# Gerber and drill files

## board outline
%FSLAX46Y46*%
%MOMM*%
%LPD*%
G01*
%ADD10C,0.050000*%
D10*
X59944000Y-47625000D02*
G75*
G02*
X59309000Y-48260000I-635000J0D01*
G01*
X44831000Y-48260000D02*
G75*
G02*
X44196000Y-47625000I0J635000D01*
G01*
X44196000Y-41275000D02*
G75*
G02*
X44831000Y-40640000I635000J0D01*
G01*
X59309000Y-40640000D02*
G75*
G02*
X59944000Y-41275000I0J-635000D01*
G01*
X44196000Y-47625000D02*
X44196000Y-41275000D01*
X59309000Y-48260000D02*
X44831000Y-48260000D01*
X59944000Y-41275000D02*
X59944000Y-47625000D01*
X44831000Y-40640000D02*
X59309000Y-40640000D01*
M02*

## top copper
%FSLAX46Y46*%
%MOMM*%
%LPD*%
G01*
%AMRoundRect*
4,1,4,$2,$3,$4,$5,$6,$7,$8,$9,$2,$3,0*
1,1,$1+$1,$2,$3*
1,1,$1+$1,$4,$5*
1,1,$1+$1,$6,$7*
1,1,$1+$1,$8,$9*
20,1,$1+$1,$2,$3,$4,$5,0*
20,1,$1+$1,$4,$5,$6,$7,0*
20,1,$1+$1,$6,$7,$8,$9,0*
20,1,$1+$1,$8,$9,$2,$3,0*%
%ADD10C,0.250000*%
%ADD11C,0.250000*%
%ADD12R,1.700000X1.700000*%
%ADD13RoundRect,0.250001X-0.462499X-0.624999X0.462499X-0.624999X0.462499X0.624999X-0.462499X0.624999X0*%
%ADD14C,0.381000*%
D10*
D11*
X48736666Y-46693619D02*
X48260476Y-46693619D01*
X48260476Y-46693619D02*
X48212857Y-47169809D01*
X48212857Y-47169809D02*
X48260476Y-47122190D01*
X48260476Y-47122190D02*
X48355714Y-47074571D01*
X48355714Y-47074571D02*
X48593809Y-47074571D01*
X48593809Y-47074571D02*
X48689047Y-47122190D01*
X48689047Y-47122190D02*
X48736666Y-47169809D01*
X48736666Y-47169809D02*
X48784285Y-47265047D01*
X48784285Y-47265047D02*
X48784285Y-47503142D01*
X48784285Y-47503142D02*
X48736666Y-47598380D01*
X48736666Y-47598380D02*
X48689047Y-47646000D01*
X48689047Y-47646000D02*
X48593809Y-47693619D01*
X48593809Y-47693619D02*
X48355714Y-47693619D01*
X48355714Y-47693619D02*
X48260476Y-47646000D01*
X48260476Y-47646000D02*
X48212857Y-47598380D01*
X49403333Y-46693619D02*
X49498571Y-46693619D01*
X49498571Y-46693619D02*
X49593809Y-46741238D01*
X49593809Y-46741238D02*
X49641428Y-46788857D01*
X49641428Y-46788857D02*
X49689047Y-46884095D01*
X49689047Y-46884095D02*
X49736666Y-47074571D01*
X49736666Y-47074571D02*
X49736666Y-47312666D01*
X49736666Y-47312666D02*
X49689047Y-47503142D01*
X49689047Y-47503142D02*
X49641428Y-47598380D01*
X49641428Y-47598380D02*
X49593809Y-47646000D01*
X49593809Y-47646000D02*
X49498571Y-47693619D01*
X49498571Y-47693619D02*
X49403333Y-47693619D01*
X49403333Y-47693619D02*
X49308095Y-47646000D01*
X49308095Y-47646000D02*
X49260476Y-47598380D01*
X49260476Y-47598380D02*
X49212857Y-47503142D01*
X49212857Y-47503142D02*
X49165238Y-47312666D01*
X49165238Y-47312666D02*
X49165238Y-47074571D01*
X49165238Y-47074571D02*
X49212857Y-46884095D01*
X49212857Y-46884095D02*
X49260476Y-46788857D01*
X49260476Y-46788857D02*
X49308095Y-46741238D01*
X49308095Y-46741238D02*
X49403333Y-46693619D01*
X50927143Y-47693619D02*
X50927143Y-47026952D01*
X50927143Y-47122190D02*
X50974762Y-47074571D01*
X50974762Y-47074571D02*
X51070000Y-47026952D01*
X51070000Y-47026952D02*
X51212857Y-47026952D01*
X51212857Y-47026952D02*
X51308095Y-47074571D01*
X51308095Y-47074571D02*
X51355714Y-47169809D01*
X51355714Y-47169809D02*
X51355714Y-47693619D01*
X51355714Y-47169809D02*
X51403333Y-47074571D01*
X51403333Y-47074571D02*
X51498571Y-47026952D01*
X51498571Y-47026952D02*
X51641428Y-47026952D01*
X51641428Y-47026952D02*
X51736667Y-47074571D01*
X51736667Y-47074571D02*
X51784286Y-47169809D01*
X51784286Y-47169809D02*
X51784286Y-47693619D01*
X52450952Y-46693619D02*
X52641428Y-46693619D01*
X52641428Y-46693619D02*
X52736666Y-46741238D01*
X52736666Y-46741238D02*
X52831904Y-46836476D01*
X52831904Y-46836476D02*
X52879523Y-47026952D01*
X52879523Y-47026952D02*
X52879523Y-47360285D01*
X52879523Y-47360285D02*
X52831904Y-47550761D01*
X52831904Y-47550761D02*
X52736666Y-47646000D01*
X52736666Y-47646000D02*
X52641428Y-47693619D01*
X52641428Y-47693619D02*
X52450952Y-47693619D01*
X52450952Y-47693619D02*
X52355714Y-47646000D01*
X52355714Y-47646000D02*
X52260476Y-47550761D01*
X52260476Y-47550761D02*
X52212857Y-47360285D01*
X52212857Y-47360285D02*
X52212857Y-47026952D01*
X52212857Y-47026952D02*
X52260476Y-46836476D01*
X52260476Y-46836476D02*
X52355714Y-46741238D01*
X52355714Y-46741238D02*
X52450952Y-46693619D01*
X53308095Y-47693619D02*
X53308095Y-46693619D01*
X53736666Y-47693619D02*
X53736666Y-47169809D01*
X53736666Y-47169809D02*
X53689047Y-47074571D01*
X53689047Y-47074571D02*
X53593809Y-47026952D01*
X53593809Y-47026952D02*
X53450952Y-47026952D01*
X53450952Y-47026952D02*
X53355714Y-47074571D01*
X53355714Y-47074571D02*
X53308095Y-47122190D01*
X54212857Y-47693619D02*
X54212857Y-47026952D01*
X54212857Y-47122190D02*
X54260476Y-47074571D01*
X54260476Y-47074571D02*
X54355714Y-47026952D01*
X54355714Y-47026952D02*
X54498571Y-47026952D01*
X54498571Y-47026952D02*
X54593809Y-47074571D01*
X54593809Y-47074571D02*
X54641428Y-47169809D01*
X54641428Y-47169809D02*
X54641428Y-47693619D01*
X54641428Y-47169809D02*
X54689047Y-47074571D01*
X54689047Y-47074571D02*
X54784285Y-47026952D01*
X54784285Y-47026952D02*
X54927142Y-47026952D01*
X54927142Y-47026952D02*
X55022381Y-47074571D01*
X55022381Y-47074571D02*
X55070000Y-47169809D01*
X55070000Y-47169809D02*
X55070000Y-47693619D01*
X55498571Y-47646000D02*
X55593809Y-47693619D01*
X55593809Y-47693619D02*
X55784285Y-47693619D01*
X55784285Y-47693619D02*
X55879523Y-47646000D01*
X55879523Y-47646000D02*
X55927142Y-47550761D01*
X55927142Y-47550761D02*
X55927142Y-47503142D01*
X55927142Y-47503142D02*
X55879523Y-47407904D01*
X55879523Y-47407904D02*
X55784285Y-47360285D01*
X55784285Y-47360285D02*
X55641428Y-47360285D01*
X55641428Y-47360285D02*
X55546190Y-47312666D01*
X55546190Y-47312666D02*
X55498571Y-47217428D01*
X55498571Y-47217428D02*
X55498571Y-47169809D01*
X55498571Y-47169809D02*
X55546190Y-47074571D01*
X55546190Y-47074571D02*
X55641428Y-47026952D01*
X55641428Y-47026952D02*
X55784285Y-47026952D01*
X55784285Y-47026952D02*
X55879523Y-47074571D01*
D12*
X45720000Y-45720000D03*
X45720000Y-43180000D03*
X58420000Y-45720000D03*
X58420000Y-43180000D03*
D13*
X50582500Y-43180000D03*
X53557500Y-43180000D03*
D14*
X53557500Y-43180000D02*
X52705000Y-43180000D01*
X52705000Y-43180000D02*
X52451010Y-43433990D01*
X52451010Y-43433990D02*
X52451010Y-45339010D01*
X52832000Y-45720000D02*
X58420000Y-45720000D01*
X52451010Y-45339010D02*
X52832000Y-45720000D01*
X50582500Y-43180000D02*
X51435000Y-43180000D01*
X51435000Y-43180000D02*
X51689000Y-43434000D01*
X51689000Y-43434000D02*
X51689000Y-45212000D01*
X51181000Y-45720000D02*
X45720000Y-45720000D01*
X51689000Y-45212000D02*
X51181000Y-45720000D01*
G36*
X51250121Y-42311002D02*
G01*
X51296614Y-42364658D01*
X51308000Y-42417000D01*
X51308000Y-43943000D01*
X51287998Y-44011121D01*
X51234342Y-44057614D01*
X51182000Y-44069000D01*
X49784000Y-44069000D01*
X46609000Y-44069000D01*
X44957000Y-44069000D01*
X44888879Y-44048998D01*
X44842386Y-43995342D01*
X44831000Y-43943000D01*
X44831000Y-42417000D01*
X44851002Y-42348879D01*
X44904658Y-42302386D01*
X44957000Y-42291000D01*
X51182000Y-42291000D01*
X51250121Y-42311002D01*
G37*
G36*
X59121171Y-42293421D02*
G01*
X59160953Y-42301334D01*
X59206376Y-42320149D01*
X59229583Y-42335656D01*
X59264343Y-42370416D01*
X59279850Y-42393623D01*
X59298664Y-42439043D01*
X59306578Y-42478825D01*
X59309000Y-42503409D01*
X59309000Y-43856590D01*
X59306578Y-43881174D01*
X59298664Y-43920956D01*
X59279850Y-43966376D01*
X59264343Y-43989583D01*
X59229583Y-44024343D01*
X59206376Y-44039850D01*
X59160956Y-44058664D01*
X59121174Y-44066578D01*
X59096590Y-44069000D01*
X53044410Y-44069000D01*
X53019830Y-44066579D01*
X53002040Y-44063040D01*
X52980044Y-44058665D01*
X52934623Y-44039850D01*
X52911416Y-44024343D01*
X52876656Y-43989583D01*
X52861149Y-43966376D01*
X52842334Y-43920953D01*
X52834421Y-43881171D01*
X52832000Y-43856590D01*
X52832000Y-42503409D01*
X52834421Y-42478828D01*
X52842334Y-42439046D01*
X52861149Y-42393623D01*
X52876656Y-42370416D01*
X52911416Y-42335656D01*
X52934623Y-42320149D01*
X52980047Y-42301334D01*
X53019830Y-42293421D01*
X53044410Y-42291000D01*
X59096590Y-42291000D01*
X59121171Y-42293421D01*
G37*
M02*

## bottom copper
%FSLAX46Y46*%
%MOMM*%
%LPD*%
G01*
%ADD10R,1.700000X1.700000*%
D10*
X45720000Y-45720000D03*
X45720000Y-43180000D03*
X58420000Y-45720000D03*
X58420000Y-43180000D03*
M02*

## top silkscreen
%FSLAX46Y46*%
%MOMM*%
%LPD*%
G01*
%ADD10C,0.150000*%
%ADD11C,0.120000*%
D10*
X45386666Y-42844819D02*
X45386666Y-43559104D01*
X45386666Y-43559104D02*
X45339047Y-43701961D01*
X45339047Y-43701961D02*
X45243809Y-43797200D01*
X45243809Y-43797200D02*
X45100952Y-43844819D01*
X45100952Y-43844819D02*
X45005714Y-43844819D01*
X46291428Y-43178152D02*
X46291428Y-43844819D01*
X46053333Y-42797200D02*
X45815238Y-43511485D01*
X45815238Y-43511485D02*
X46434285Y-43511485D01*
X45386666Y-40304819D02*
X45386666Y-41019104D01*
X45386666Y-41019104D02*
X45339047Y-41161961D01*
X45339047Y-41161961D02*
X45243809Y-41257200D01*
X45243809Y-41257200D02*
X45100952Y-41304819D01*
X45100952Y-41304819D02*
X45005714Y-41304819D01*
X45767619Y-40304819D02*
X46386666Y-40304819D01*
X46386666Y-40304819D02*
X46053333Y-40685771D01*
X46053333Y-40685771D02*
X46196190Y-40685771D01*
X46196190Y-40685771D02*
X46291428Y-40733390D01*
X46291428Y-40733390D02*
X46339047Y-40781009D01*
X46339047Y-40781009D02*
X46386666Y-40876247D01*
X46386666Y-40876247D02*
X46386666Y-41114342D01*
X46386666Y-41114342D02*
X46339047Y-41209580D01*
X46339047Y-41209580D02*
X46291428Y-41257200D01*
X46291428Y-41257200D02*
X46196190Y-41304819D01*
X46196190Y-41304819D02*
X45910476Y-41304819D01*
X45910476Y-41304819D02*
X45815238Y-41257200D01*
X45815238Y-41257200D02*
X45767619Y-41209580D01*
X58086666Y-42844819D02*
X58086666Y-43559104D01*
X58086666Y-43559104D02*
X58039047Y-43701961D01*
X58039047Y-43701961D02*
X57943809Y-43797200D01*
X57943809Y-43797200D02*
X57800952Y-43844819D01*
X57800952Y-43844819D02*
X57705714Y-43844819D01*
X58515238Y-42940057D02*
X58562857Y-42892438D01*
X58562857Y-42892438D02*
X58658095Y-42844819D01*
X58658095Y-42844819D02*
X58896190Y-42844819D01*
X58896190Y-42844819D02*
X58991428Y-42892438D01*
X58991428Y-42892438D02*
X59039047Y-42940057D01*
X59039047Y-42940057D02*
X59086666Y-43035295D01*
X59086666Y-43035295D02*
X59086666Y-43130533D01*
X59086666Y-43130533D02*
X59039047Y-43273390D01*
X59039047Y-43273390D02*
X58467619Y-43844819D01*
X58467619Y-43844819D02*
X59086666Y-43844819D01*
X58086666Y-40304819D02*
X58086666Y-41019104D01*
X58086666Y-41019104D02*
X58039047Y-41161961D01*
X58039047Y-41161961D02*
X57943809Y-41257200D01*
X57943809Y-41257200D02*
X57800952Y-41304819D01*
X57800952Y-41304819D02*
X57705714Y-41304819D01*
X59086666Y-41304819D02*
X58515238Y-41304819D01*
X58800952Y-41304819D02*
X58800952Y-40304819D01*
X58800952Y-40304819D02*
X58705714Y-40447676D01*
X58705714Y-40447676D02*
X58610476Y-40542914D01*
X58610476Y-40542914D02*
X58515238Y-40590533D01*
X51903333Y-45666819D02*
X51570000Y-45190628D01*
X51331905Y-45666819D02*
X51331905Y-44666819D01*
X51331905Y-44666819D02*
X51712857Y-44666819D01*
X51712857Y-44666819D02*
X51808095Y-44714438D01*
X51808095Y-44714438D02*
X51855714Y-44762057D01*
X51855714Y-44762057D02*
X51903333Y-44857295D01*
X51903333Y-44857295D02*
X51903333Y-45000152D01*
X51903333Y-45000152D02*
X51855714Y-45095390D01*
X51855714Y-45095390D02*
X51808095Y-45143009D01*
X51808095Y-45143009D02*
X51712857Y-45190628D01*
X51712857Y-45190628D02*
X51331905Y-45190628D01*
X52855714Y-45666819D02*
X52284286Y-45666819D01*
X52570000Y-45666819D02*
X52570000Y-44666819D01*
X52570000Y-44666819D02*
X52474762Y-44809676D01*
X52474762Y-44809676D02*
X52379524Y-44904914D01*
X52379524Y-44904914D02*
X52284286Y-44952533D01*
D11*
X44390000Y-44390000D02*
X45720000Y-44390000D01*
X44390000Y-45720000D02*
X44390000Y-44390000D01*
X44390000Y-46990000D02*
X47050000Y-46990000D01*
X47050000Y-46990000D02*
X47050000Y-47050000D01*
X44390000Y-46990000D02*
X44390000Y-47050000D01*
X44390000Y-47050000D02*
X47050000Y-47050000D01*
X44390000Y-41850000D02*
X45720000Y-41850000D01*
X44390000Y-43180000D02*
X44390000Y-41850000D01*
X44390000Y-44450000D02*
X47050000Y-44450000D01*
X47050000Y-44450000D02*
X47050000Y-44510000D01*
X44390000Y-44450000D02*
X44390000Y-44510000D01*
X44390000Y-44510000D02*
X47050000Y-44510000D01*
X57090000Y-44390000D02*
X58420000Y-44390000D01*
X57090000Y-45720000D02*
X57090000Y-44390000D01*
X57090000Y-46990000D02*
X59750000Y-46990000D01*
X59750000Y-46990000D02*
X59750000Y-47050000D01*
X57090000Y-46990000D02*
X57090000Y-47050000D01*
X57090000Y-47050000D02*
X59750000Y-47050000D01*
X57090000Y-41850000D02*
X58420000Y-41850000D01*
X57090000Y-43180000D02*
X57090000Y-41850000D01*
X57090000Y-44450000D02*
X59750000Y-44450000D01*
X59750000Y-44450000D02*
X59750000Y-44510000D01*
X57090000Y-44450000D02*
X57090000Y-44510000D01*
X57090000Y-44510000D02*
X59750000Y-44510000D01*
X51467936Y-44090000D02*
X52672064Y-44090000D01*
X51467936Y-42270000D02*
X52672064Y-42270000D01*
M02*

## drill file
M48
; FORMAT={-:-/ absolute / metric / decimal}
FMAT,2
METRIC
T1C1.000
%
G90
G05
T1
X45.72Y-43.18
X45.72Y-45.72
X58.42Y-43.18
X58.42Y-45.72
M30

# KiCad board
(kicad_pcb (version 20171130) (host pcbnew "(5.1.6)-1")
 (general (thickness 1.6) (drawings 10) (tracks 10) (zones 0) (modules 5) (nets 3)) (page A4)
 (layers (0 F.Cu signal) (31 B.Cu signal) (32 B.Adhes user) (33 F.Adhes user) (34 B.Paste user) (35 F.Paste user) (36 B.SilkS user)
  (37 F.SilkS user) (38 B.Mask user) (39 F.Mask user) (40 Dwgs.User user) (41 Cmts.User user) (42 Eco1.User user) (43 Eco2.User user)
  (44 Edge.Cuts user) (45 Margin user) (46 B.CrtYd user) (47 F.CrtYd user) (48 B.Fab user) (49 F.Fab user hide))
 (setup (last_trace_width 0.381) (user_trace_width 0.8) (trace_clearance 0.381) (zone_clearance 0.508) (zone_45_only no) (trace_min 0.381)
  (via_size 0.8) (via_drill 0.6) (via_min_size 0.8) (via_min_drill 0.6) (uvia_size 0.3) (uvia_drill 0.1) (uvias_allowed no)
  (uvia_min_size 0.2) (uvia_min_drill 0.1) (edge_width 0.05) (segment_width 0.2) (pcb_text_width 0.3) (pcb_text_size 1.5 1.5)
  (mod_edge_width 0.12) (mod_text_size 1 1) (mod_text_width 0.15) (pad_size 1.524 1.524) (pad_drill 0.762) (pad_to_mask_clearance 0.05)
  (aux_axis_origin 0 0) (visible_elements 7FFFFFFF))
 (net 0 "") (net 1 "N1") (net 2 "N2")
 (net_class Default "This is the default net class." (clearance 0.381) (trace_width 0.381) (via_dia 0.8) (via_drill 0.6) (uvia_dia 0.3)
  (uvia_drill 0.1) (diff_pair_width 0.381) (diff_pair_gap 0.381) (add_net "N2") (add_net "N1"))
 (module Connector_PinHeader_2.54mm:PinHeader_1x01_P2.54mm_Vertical (layer F.Cu) (at 45.72 45.72)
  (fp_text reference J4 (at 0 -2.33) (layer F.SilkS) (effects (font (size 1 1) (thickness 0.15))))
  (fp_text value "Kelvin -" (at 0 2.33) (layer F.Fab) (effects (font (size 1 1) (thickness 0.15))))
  (fp_line (start -1.33 -1.33) (end 0 -1.33) (layer F.SilkS) (width 0.12))
  (fp_line (start -1.33 0) (end -1.33 -1.33) (layer F.SilkS) (width 0.12))
  (fp_line (start -1.33 1.27) (end 1.33 1.27) (layer F.SilkS) (width 0.12))
  (fp_line (start 1.33 1.27) (end 1.33 1.33) (layer F.SilkS) (width 0.12))
  (fp_line (start -1.33 1.27) (end -1.33 1.33) (layer F.SilkS) (width 0.12))
  (fp_line (start -1.33 1.33) (end 1.33 1.33) (layer F.SilkS) (width 0.12))
  (pad 1 thru_hole rect (at 0 0) (size 1.7 1.7) (drill 1) (layers *.Cu *.Mask) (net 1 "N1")))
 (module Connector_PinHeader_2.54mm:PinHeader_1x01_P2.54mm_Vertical (layer F.Cu) (at 45.72 43.18)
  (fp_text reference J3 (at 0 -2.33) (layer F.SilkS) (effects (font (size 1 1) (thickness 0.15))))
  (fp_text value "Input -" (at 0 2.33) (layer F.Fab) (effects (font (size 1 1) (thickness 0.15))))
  (fp_line (start -1.33 -1.33) (end 0 -1.33) (layer F.SilkS) (width 0.12))
  (fp_line (start -1.33 0) (end -1.33 -1.33) (layer F.SilkS) (width 0.12))
  (fp_line (start -1.33 1.27) (end 1.33 1.27) (layer F.SilkS) (width 0.12))
  (fp_line (start 1.33 1.27) (end 1.33 1.33) (layer F.SilkS) (width 0.12))
  (fp_line (start -1.33 1.27) (end -1.33 1.33) (layer F.SilkS) (width 0.12))
  (fp_line (start -1.33 1.33) (end 1.33 1.33) (layer F.SilkS) (width 0.12))
  (pad 1 thru_hole rect (at 0 0) (size 1.7 1.7) (drill 1) (layers *.Cu *.Mask) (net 1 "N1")))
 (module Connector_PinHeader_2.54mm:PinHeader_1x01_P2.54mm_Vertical (layer F.Cu) (at 58.42 45.72)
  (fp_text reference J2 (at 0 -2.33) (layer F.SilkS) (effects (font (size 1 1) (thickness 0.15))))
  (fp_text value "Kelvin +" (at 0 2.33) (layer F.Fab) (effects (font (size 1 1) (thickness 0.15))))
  (fp_line (start -1.33 -1.33) (end 0 -1.33) (layer F.SilkS) (width 0.12))
  (fp_line (start -1.33 0) (end -1.33 -1.33) (layer F.SilkS) (width 0.12))
  (fp_line (start -1.33 1.27) (end 1.33 1.27) (layer F.SilkS) (width 0.12))
  (fp_line (start 1.33 1.27) (end 1.33 1.33) (layer F.SilkS) (width 0.12))
  (fp_line (start -1.33 1.27) (end -1.33 1.33) (layer F.SilkS) (width 0.12))
  (fp_line (start -1.33 1.33) (end 1.33 1.33) (layer F.SilkS) (width 0.12))
  (pad 1 thru_hole rect (at 0 0) (size 1.7 1.7) (drill 1) (layers *.Cu *.Mask) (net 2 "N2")))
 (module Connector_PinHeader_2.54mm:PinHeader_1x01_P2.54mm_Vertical (layer F.Cu) (at 58.42 43.18)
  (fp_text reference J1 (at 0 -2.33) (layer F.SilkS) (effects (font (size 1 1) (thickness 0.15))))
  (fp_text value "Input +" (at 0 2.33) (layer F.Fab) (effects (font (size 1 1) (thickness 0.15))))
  (fp_line (start -1.33 -1.33) (end 0 -1.33) (layer F.SilkS) (width 0.12))
  (fp_line (start -1.33 0) (end -1.33 -1.33) (layer F.SilkS) (width 0.12))
  (fp_line (start -1.33 1.27) (end 1.33 1.27) (layer F.SilkS) (width 0.12))
  (fp_line (start 1.33 1.27) (end 1.33 1.33) (layer F.SilkS) (width 0.12))
  (fp_line (start -1.33 1.27) (end -1.33 1.33) (layer F.SilkS) (width 0.12))
  (fp_line (start -1.33 1.33) (end 1.33 1.33) (layer F.SilkS) (width 0.12))
  (pad 1 thru_hole rect (at 0 0) (size 1.7 1.7) (drill 1) (layers *.Cu *.Mask) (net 2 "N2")))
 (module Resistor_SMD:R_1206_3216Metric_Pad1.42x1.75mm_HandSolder (layer F.Cu) (at 52.07 43.18)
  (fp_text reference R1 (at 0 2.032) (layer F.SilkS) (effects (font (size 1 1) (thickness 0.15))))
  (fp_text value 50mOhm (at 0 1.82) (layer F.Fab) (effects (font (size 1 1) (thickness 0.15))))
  (fp_line (start -0.602064 0.91) (end 0.602064 0.91) (layer F.SilkS) (width 0.12))
  (fp_line (start -0.602064 -0.91) (end 0.602064 -0.91) (layer F.SilkS) (width 0.12))
  (pad 1 smd roundrect (at -1.4875 0) (size 1.425 1.75) (layers F.Cu F.Paste F.Mask) (roundrect_rratio 0.175439) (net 1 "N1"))
  (pad 2 smd roundrect (at 1.4875 0) (size 1.425 1.75) (layers F.Cu F.Paste F.Mask) (roundrect_rratio 0.175439) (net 2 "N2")))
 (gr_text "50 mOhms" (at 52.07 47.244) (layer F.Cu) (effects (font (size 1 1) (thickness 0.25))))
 (gr_arc (start 59.309 47.625) (end 59.309 48.26) (angle -90) (layer Edge.Cuts) (width 0.05))
 (gr_arc (start 44.831 47.625) (end 44.196 47.625) (angle -90) (layer Edge.Cuts) (width 0.05))
 (gr_arc (start 44.831 41.275) (end 44.831 40.64) (angle -90) (layer Edge.Cuts) (width 0.05))
 (gr_arc (start 59.309 41.275) (end 59.944 41.275) (angle -90) (layer Edge.Cuts) (width 0.05))
 (gr_line (start 44.196 47.625) (end 44.196 41.275) (layer Edge.Cuts) (width 0.05))
 (gr_line (start 59.309 48.26) (end 44.831 48.26) (layer Edge.Cuts) (width 0.05))
 (gr_line (start 59.944 41.275) (end 59.944 47.625) (layer Edge.Cuts) (width 0.05))
 (gr_line (start 44.831 40.64) (end 59.309 40.64) (layer Edge.Cuts) (width 0.05))
 (segment (start 53.5575 43.18) (end 52.705 43.18) (width 0.381) (layer F.Cu) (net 2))
 (segment (start 52.705 43.18) (end 52.45101 43.43399) (width 0.381) (layer F.Cu) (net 2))
 (segment (start 52.45101 43.43399) (end 52.45101 45.33901) (width 0.381) (layer F.Cu) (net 2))
 (segment (start 52.832 45.72) (end 58.42 45.72) (width 0.381) (layer F.Cu) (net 2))
 (segment (start 52.45101 45.33901) (end 52.832 45.72) (width 0.381) (layer F.Cu) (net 2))
 (segment (start 50.5825 43.18) (end 51.435 43.18) (width 0.381) (layer F.Cu) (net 1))
 (segment (start 51.435 43.18) (end 51.689 43.434) (width 0.381) (layer F.Cu) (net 1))
 (segment (start 51.689 43.434) (end 51.689 45.212) (width 0.381) (layer F.Cu) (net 1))
 (segment (start 51.181 45.72) (end 45.72 45.72) (width 0.381) (layer F.Cu) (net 1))
 (segment (start 51.689 45.212) (end 51.181 45.72) (width 0.381) (layer F.Cu) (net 1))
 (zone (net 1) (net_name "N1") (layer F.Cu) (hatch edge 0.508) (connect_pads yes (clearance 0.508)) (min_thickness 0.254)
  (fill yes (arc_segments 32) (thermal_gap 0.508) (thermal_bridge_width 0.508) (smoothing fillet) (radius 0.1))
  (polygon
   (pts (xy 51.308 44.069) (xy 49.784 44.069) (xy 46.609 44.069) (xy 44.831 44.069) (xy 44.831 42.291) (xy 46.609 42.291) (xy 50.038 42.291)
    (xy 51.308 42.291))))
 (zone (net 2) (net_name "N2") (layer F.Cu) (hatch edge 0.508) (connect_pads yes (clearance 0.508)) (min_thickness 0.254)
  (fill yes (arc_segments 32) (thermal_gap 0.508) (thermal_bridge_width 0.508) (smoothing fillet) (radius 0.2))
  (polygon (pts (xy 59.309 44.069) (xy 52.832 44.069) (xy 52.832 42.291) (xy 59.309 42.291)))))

